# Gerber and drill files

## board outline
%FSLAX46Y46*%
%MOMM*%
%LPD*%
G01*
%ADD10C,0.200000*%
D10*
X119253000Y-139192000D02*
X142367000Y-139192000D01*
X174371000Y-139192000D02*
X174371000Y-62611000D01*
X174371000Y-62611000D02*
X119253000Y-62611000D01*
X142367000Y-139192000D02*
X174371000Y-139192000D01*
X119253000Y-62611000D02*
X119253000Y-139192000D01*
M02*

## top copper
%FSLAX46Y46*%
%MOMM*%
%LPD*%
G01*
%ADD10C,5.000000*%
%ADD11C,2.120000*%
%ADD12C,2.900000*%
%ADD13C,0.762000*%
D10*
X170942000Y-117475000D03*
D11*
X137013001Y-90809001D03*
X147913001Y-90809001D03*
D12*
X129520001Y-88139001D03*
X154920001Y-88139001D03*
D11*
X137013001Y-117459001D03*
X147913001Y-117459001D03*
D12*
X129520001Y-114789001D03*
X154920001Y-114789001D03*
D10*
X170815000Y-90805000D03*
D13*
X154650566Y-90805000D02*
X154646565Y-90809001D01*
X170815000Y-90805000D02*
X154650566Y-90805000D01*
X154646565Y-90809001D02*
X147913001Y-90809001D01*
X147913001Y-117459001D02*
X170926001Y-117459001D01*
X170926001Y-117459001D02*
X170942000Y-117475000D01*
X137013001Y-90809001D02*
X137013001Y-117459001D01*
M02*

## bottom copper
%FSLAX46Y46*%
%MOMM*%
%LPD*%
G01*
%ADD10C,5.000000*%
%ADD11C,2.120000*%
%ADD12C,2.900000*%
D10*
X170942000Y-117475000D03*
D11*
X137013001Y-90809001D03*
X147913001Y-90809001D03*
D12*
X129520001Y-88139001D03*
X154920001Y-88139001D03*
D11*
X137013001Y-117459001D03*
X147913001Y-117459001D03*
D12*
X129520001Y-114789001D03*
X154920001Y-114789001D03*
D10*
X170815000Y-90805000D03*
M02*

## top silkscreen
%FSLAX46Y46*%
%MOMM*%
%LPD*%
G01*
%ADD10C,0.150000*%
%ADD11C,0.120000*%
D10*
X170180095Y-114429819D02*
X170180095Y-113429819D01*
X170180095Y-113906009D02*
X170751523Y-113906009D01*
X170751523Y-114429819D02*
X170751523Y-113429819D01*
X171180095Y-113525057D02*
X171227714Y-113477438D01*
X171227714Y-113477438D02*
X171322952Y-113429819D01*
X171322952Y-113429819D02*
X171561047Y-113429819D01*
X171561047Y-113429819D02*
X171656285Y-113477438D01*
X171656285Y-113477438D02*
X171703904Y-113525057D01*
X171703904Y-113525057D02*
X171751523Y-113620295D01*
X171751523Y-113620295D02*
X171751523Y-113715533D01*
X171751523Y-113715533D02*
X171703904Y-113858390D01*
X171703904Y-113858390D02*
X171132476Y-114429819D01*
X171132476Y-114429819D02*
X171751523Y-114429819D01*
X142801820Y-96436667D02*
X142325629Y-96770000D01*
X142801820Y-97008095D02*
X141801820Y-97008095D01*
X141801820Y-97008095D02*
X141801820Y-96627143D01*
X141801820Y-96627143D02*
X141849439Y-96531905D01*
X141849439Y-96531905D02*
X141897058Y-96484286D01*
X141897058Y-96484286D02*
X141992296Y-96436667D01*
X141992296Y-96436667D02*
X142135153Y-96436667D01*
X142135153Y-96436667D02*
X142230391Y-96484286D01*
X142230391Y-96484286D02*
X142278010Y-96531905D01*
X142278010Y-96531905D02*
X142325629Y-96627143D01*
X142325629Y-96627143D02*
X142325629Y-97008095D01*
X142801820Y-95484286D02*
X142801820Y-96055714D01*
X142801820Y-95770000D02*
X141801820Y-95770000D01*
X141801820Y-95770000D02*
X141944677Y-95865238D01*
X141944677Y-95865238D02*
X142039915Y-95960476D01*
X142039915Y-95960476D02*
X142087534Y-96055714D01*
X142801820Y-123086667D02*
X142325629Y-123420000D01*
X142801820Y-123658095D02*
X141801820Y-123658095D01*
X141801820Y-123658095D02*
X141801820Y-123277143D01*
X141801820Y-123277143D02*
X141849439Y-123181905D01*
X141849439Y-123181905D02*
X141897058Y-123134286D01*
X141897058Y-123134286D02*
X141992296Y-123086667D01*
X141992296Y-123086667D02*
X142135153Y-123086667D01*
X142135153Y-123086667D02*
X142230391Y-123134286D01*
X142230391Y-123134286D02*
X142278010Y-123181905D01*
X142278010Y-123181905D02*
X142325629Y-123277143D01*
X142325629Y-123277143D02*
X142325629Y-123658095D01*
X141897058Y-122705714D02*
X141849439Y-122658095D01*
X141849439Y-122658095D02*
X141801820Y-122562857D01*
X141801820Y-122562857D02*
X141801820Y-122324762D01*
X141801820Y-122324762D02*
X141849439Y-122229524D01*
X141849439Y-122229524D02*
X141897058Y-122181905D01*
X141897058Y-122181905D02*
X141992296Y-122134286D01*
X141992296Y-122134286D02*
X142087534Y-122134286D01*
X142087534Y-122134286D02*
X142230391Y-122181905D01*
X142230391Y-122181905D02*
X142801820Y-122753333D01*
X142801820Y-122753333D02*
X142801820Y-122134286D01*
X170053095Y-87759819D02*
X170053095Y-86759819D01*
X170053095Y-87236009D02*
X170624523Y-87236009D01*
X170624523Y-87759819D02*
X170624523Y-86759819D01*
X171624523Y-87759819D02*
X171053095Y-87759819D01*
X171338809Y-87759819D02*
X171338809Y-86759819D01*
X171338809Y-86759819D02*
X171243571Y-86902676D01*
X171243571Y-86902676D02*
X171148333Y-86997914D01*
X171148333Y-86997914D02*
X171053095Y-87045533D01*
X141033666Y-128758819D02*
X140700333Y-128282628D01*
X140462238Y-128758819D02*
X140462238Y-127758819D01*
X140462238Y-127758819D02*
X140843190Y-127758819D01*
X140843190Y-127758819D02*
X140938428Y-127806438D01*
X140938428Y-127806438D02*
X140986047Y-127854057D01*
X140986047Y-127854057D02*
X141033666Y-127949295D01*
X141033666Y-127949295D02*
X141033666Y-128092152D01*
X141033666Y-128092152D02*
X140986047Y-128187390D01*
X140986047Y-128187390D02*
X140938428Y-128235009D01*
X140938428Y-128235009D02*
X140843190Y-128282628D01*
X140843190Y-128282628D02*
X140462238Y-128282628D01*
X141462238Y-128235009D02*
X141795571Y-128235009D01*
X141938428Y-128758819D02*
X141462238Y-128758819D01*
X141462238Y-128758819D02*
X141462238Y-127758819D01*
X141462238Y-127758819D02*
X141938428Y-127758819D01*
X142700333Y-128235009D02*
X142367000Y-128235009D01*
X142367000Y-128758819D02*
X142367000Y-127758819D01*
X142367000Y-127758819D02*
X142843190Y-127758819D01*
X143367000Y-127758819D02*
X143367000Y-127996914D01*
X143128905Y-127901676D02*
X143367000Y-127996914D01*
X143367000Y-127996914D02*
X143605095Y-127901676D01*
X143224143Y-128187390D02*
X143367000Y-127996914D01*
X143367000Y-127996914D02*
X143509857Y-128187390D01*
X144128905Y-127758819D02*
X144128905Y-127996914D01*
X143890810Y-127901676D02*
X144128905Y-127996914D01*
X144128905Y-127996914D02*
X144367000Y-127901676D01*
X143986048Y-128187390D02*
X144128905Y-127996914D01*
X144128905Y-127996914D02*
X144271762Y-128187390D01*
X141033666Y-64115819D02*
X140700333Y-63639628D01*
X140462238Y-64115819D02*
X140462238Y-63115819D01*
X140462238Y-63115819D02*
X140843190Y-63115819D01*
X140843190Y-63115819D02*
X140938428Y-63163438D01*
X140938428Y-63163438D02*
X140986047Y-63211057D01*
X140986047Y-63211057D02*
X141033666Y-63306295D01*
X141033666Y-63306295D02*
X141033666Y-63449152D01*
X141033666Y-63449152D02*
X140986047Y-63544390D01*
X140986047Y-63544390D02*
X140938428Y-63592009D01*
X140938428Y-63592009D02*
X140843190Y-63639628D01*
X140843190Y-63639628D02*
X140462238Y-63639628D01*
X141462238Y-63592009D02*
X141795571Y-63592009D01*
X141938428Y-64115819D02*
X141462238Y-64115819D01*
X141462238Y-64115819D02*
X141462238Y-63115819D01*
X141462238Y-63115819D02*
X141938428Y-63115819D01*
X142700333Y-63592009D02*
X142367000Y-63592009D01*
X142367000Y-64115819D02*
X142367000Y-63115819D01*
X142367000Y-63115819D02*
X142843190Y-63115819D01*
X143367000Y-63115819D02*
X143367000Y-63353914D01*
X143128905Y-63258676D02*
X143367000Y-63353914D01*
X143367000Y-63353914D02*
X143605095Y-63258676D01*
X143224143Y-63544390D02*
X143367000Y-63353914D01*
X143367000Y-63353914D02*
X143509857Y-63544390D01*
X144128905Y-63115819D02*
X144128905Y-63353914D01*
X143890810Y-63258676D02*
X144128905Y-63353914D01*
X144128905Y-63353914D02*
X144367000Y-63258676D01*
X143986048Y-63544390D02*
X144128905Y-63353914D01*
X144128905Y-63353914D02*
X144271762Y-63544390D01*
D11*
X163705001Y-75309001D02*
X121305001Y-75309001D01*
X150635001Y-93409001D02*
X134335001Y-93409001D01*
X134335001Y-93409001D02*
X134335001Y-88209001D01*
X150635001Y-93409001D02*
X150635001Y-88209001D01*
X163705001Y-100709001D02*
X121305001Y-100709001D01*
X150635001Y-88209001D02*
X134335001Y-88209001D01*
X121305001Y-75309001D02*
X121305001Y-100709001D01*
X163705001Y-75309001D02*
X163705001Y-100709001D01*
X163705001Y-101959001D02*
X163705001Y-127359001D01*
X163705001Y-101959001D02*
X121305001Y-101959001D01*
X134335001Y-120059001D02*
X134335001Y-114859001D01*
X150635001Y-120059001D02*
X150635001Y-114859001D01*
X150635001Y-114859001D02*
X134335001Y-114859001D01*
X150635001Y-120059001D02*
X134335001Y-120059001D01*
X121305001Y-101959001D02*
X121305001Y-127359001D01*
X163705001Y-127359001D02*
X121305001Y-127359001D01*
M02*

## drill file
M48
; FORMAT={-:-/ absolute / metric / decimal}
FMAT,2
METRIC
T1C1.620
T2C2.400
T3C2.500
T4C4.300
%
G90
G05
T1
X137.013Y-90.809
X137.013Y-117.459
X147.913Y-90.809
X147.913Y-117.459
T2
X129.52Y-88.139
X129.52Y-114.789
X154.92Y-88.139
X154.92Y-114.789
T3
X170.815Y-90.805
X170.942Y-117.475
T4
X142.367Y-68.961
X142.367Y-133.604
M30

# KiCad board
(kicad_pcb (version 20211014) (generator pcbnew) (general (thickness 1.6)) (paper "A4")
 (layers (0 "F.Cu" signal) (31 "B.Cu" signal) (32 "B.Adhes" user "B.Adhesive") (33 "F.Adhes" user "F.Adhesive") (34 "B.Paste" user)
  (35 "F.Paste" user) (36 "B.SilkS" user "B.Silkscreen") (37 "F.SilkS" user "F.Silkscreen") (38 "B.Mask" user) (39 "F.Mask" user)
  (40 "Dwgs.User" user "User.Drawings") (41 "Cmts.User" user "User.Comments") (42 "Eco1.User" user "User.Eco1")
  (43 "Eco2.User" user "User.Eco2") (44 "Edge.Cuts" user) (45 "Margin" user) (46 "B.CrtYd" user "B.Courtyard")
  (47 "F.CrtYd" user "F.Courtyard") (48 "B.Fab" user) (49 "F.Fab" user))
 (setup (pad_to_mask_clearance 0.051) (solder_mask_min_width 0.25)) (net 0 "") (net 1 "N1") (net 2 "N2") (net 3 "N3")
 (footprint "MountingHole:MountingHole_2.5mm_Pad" (layer "F.Cu") (at 170.942 117.475)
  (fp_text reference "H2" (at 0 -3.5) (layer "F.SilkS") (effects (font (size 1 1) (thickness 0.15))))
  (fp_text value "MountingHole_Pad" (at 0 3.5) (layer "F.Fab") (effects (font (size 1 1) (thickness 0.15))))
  (pad "1" thru_hole circle locked (at 0 0) (size 5 5) (drill 2.5) (layers *.Cu *.Mask) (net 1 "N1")))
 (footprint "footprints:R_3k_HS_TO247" (layer "F.Cu") (at 137.013001 90.809001)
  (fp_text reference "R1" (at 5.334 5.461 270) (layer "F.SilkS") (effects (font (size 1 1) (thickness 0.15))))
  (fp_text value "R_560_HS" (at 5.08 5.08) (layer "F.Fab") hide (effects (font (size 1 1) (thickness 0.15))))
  (fp_line (start 26.692 -15.5) (end -15.708 -15.5) (layer "F.SilkS") (width 0.12))
  (fp_line (start 13.622 2.6) (end -2.678 2.6) (layer "F.SilkS") (width 0.12))
  (fp_line (start -2.678 2.6) (end -2.678 -2.6) (layer "F.SilkS") (width 0.12))
  (fp_line (start 13.622 2.6) (end 13.622 -2.6) (layer "F.SilkS") (width 0.12))
  (fp_line (start 26.692 9.9) (end -15.708 9.9) (layer "F.SilkS") (width 0.12))
  (fp_line (start 13.622 -2.6) (end -2.678 -2.6) (layer "F.SilkS") (width 0.12))
  (fp_line (start -15.708 -15.5) (end -15.708 9.9) (layer "F.SilkS") (width 0.12))
  (fp_line (start 26.692 -15.5) (end 26.692 9.9) (layer "F.SilkS") (width 0.12))
  (pad "1" thru_hole circle locked (at 0 0) (size 2.12 2.12) (drill 1.62) (layers *.Cu *.Mask) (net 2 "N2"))
  (pad "2" thru_hole circle locked (at 10.9 0) (size 2.12 2.12) (drill 1.62) (layers *.Cu *.Mask) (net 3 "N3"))
  (pad "4" thru_hole circle locked (at -7.493 -2.67) (size 2.9 2.9) (drill 2.4) (layers *.Cu *.Mask))
  (pad "5" thru_hole circle locked (at 17.907 -2.67) (size 2.9 2.9) (drill 2.4) (layers *.Cu *.Mask)))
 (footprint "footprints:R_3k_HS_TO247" (layer "F.Cu") (at 137.013001 117.459001)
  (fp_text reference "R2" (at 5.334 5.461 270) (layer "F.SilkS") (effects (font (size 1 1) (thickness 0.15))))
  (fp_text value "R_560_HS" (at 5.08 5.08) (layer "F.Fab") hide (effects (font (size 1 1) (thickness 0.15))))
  (fp_line (start 26.692 -15.5) (end 26.692 9.9) (layer "F.SilkS") (width 0.12))
  (fp_line (start 26.692 -15.5) (end -15.708 -15.5) (layer "F.SilkS") (width 0.12))
  (fp_line (start -2.678 2.6) (end -2.678 -2.6) (layer "F.SilkS") (width 0.12))
  (fp_line (start 13.622 2.6) (end 13.622 -2.6) (layer "F.SilkS") (width 0.12))
  (fp_line (start 13.622 -2.6) (end -2.678 -2.6) (layer "F.SilkS") (width 0.12))
  (fp_line (start 13.622 2.6) (end -2.678 2.6) (layer "F.SilkS") (width 0.12))
  (fp_line (start -15.708 -15.5) (end -15.708 9.9) (layer "F.SilkS") (width 0.12))
  (fp_line (start 26.692 9.9) (end -15.708 9.9) (layer "F.SilkS") (width 0.12))
  (pad "1" thru_hole circle locked (at 0 0) (size 2.12 2.12) (drill 1.62) (layers *.Cu *.Mask) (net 2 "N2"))
  (pad "2" thru_hole circle locked (at 10.9 0) (size 2.12 2.12) (drill 1.62) (layers *.Cu *.Mask) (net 1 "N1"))
  (pad "4" thru_hole circle locked (at -7.493 -2.67) (size 2.9 2.9) (drill 2.4) (layers *.Cu *.Mask))
  (pad "5" thru_hole circle locked (at 17.907 -2.67) (size 2.9 2.9) (drill 2.4) (layers *.Cu *.Mask)))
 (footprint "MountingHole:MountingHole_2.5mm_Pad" (layer "F.Cu") (at 170.815 90.805)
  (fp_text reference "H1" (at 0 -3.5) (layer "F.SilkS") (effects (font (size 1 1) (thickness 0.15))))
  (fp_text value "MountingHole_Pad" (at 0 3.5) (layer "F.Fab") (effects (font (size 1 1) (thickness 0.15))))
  (pad "1" thru_hole circle locked (at 0 0) (size 5 5) (drill 2.5) (layers *.Cu *.Mask) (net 3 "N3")))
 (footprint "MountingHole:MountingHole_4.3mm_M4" (layer "F.Cu") (at 142.367 133.604)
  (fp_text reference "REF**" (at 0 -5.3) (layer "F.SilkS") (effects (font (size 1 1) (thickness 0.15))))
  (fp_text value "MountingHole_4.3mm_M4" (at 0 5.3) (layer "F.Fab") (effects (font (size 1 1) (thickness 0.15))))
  (pad "" np_thru_hole circle locked (at 0 0) (size 4.3 4.3) (drill 4.3) (layers *.Cu *.Mask)))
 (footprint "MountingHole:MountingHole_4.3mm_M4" (layer "F.Cu") (at 142.367 68.961)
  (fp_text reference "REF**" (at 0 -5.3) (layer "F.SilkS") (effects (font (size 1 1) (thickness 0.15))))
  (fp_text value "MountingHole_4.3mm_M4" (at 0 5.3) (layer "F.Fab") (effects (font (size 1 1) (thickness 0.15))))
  (pad "" np_thru_hole circle locked (at 0 0) (size 4.3 4.3) (drill 4.3) (layers *.Cu *.Mask)))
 (gr_line (start 119.253 139.192) (end 142.367 139.192) (layer "Edge.Cuts") (width 0.2))
 (gr_line (start 174.371 139.192) (end 174.371 62.611) (layer "Edge.Cuts") (width 0.2))
 (gr_line (start 174.371 62.611) (end 119.253 62.611) (layer "Edge.Cuts") (width 0.2))
 (gr_line (start 142.367 139.192) (end 174.371 139.192) (layer "Edge.Cuts") (width 0.2))
 (gr_line (start 119.253 62.611) (end 119.253 139.192) (layer "Edge.Cuts") (width 0.2))
 (segment (start 154.650566 90.805) (end 154.646565 90.809001) (width 0.762) (layer "F.Cu") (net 3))
 (segment (start 170.815 90.805) (end 154.650566 90.805) (width 0.762) (layer "F.Cu") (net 3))
 (segment (start 154.646565 90.809001) (end 147.913001 90.809001) (width 0.762) (layer "F.Cu") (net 3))
 (segment (start 147.913001 117.459001) (end 170.926001 117.459001) (width 0.762) (layer "F.Cu") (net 1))
 (segment (start 170.926001 117.459001) (end 170.942 117.475) (width 0.762) (layer "F.Cu") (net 1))
 (segment (start 137.013001 90.809001) (end 137.013001 117.459001) (width 0.762) (layer "F.Cu") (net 2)))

